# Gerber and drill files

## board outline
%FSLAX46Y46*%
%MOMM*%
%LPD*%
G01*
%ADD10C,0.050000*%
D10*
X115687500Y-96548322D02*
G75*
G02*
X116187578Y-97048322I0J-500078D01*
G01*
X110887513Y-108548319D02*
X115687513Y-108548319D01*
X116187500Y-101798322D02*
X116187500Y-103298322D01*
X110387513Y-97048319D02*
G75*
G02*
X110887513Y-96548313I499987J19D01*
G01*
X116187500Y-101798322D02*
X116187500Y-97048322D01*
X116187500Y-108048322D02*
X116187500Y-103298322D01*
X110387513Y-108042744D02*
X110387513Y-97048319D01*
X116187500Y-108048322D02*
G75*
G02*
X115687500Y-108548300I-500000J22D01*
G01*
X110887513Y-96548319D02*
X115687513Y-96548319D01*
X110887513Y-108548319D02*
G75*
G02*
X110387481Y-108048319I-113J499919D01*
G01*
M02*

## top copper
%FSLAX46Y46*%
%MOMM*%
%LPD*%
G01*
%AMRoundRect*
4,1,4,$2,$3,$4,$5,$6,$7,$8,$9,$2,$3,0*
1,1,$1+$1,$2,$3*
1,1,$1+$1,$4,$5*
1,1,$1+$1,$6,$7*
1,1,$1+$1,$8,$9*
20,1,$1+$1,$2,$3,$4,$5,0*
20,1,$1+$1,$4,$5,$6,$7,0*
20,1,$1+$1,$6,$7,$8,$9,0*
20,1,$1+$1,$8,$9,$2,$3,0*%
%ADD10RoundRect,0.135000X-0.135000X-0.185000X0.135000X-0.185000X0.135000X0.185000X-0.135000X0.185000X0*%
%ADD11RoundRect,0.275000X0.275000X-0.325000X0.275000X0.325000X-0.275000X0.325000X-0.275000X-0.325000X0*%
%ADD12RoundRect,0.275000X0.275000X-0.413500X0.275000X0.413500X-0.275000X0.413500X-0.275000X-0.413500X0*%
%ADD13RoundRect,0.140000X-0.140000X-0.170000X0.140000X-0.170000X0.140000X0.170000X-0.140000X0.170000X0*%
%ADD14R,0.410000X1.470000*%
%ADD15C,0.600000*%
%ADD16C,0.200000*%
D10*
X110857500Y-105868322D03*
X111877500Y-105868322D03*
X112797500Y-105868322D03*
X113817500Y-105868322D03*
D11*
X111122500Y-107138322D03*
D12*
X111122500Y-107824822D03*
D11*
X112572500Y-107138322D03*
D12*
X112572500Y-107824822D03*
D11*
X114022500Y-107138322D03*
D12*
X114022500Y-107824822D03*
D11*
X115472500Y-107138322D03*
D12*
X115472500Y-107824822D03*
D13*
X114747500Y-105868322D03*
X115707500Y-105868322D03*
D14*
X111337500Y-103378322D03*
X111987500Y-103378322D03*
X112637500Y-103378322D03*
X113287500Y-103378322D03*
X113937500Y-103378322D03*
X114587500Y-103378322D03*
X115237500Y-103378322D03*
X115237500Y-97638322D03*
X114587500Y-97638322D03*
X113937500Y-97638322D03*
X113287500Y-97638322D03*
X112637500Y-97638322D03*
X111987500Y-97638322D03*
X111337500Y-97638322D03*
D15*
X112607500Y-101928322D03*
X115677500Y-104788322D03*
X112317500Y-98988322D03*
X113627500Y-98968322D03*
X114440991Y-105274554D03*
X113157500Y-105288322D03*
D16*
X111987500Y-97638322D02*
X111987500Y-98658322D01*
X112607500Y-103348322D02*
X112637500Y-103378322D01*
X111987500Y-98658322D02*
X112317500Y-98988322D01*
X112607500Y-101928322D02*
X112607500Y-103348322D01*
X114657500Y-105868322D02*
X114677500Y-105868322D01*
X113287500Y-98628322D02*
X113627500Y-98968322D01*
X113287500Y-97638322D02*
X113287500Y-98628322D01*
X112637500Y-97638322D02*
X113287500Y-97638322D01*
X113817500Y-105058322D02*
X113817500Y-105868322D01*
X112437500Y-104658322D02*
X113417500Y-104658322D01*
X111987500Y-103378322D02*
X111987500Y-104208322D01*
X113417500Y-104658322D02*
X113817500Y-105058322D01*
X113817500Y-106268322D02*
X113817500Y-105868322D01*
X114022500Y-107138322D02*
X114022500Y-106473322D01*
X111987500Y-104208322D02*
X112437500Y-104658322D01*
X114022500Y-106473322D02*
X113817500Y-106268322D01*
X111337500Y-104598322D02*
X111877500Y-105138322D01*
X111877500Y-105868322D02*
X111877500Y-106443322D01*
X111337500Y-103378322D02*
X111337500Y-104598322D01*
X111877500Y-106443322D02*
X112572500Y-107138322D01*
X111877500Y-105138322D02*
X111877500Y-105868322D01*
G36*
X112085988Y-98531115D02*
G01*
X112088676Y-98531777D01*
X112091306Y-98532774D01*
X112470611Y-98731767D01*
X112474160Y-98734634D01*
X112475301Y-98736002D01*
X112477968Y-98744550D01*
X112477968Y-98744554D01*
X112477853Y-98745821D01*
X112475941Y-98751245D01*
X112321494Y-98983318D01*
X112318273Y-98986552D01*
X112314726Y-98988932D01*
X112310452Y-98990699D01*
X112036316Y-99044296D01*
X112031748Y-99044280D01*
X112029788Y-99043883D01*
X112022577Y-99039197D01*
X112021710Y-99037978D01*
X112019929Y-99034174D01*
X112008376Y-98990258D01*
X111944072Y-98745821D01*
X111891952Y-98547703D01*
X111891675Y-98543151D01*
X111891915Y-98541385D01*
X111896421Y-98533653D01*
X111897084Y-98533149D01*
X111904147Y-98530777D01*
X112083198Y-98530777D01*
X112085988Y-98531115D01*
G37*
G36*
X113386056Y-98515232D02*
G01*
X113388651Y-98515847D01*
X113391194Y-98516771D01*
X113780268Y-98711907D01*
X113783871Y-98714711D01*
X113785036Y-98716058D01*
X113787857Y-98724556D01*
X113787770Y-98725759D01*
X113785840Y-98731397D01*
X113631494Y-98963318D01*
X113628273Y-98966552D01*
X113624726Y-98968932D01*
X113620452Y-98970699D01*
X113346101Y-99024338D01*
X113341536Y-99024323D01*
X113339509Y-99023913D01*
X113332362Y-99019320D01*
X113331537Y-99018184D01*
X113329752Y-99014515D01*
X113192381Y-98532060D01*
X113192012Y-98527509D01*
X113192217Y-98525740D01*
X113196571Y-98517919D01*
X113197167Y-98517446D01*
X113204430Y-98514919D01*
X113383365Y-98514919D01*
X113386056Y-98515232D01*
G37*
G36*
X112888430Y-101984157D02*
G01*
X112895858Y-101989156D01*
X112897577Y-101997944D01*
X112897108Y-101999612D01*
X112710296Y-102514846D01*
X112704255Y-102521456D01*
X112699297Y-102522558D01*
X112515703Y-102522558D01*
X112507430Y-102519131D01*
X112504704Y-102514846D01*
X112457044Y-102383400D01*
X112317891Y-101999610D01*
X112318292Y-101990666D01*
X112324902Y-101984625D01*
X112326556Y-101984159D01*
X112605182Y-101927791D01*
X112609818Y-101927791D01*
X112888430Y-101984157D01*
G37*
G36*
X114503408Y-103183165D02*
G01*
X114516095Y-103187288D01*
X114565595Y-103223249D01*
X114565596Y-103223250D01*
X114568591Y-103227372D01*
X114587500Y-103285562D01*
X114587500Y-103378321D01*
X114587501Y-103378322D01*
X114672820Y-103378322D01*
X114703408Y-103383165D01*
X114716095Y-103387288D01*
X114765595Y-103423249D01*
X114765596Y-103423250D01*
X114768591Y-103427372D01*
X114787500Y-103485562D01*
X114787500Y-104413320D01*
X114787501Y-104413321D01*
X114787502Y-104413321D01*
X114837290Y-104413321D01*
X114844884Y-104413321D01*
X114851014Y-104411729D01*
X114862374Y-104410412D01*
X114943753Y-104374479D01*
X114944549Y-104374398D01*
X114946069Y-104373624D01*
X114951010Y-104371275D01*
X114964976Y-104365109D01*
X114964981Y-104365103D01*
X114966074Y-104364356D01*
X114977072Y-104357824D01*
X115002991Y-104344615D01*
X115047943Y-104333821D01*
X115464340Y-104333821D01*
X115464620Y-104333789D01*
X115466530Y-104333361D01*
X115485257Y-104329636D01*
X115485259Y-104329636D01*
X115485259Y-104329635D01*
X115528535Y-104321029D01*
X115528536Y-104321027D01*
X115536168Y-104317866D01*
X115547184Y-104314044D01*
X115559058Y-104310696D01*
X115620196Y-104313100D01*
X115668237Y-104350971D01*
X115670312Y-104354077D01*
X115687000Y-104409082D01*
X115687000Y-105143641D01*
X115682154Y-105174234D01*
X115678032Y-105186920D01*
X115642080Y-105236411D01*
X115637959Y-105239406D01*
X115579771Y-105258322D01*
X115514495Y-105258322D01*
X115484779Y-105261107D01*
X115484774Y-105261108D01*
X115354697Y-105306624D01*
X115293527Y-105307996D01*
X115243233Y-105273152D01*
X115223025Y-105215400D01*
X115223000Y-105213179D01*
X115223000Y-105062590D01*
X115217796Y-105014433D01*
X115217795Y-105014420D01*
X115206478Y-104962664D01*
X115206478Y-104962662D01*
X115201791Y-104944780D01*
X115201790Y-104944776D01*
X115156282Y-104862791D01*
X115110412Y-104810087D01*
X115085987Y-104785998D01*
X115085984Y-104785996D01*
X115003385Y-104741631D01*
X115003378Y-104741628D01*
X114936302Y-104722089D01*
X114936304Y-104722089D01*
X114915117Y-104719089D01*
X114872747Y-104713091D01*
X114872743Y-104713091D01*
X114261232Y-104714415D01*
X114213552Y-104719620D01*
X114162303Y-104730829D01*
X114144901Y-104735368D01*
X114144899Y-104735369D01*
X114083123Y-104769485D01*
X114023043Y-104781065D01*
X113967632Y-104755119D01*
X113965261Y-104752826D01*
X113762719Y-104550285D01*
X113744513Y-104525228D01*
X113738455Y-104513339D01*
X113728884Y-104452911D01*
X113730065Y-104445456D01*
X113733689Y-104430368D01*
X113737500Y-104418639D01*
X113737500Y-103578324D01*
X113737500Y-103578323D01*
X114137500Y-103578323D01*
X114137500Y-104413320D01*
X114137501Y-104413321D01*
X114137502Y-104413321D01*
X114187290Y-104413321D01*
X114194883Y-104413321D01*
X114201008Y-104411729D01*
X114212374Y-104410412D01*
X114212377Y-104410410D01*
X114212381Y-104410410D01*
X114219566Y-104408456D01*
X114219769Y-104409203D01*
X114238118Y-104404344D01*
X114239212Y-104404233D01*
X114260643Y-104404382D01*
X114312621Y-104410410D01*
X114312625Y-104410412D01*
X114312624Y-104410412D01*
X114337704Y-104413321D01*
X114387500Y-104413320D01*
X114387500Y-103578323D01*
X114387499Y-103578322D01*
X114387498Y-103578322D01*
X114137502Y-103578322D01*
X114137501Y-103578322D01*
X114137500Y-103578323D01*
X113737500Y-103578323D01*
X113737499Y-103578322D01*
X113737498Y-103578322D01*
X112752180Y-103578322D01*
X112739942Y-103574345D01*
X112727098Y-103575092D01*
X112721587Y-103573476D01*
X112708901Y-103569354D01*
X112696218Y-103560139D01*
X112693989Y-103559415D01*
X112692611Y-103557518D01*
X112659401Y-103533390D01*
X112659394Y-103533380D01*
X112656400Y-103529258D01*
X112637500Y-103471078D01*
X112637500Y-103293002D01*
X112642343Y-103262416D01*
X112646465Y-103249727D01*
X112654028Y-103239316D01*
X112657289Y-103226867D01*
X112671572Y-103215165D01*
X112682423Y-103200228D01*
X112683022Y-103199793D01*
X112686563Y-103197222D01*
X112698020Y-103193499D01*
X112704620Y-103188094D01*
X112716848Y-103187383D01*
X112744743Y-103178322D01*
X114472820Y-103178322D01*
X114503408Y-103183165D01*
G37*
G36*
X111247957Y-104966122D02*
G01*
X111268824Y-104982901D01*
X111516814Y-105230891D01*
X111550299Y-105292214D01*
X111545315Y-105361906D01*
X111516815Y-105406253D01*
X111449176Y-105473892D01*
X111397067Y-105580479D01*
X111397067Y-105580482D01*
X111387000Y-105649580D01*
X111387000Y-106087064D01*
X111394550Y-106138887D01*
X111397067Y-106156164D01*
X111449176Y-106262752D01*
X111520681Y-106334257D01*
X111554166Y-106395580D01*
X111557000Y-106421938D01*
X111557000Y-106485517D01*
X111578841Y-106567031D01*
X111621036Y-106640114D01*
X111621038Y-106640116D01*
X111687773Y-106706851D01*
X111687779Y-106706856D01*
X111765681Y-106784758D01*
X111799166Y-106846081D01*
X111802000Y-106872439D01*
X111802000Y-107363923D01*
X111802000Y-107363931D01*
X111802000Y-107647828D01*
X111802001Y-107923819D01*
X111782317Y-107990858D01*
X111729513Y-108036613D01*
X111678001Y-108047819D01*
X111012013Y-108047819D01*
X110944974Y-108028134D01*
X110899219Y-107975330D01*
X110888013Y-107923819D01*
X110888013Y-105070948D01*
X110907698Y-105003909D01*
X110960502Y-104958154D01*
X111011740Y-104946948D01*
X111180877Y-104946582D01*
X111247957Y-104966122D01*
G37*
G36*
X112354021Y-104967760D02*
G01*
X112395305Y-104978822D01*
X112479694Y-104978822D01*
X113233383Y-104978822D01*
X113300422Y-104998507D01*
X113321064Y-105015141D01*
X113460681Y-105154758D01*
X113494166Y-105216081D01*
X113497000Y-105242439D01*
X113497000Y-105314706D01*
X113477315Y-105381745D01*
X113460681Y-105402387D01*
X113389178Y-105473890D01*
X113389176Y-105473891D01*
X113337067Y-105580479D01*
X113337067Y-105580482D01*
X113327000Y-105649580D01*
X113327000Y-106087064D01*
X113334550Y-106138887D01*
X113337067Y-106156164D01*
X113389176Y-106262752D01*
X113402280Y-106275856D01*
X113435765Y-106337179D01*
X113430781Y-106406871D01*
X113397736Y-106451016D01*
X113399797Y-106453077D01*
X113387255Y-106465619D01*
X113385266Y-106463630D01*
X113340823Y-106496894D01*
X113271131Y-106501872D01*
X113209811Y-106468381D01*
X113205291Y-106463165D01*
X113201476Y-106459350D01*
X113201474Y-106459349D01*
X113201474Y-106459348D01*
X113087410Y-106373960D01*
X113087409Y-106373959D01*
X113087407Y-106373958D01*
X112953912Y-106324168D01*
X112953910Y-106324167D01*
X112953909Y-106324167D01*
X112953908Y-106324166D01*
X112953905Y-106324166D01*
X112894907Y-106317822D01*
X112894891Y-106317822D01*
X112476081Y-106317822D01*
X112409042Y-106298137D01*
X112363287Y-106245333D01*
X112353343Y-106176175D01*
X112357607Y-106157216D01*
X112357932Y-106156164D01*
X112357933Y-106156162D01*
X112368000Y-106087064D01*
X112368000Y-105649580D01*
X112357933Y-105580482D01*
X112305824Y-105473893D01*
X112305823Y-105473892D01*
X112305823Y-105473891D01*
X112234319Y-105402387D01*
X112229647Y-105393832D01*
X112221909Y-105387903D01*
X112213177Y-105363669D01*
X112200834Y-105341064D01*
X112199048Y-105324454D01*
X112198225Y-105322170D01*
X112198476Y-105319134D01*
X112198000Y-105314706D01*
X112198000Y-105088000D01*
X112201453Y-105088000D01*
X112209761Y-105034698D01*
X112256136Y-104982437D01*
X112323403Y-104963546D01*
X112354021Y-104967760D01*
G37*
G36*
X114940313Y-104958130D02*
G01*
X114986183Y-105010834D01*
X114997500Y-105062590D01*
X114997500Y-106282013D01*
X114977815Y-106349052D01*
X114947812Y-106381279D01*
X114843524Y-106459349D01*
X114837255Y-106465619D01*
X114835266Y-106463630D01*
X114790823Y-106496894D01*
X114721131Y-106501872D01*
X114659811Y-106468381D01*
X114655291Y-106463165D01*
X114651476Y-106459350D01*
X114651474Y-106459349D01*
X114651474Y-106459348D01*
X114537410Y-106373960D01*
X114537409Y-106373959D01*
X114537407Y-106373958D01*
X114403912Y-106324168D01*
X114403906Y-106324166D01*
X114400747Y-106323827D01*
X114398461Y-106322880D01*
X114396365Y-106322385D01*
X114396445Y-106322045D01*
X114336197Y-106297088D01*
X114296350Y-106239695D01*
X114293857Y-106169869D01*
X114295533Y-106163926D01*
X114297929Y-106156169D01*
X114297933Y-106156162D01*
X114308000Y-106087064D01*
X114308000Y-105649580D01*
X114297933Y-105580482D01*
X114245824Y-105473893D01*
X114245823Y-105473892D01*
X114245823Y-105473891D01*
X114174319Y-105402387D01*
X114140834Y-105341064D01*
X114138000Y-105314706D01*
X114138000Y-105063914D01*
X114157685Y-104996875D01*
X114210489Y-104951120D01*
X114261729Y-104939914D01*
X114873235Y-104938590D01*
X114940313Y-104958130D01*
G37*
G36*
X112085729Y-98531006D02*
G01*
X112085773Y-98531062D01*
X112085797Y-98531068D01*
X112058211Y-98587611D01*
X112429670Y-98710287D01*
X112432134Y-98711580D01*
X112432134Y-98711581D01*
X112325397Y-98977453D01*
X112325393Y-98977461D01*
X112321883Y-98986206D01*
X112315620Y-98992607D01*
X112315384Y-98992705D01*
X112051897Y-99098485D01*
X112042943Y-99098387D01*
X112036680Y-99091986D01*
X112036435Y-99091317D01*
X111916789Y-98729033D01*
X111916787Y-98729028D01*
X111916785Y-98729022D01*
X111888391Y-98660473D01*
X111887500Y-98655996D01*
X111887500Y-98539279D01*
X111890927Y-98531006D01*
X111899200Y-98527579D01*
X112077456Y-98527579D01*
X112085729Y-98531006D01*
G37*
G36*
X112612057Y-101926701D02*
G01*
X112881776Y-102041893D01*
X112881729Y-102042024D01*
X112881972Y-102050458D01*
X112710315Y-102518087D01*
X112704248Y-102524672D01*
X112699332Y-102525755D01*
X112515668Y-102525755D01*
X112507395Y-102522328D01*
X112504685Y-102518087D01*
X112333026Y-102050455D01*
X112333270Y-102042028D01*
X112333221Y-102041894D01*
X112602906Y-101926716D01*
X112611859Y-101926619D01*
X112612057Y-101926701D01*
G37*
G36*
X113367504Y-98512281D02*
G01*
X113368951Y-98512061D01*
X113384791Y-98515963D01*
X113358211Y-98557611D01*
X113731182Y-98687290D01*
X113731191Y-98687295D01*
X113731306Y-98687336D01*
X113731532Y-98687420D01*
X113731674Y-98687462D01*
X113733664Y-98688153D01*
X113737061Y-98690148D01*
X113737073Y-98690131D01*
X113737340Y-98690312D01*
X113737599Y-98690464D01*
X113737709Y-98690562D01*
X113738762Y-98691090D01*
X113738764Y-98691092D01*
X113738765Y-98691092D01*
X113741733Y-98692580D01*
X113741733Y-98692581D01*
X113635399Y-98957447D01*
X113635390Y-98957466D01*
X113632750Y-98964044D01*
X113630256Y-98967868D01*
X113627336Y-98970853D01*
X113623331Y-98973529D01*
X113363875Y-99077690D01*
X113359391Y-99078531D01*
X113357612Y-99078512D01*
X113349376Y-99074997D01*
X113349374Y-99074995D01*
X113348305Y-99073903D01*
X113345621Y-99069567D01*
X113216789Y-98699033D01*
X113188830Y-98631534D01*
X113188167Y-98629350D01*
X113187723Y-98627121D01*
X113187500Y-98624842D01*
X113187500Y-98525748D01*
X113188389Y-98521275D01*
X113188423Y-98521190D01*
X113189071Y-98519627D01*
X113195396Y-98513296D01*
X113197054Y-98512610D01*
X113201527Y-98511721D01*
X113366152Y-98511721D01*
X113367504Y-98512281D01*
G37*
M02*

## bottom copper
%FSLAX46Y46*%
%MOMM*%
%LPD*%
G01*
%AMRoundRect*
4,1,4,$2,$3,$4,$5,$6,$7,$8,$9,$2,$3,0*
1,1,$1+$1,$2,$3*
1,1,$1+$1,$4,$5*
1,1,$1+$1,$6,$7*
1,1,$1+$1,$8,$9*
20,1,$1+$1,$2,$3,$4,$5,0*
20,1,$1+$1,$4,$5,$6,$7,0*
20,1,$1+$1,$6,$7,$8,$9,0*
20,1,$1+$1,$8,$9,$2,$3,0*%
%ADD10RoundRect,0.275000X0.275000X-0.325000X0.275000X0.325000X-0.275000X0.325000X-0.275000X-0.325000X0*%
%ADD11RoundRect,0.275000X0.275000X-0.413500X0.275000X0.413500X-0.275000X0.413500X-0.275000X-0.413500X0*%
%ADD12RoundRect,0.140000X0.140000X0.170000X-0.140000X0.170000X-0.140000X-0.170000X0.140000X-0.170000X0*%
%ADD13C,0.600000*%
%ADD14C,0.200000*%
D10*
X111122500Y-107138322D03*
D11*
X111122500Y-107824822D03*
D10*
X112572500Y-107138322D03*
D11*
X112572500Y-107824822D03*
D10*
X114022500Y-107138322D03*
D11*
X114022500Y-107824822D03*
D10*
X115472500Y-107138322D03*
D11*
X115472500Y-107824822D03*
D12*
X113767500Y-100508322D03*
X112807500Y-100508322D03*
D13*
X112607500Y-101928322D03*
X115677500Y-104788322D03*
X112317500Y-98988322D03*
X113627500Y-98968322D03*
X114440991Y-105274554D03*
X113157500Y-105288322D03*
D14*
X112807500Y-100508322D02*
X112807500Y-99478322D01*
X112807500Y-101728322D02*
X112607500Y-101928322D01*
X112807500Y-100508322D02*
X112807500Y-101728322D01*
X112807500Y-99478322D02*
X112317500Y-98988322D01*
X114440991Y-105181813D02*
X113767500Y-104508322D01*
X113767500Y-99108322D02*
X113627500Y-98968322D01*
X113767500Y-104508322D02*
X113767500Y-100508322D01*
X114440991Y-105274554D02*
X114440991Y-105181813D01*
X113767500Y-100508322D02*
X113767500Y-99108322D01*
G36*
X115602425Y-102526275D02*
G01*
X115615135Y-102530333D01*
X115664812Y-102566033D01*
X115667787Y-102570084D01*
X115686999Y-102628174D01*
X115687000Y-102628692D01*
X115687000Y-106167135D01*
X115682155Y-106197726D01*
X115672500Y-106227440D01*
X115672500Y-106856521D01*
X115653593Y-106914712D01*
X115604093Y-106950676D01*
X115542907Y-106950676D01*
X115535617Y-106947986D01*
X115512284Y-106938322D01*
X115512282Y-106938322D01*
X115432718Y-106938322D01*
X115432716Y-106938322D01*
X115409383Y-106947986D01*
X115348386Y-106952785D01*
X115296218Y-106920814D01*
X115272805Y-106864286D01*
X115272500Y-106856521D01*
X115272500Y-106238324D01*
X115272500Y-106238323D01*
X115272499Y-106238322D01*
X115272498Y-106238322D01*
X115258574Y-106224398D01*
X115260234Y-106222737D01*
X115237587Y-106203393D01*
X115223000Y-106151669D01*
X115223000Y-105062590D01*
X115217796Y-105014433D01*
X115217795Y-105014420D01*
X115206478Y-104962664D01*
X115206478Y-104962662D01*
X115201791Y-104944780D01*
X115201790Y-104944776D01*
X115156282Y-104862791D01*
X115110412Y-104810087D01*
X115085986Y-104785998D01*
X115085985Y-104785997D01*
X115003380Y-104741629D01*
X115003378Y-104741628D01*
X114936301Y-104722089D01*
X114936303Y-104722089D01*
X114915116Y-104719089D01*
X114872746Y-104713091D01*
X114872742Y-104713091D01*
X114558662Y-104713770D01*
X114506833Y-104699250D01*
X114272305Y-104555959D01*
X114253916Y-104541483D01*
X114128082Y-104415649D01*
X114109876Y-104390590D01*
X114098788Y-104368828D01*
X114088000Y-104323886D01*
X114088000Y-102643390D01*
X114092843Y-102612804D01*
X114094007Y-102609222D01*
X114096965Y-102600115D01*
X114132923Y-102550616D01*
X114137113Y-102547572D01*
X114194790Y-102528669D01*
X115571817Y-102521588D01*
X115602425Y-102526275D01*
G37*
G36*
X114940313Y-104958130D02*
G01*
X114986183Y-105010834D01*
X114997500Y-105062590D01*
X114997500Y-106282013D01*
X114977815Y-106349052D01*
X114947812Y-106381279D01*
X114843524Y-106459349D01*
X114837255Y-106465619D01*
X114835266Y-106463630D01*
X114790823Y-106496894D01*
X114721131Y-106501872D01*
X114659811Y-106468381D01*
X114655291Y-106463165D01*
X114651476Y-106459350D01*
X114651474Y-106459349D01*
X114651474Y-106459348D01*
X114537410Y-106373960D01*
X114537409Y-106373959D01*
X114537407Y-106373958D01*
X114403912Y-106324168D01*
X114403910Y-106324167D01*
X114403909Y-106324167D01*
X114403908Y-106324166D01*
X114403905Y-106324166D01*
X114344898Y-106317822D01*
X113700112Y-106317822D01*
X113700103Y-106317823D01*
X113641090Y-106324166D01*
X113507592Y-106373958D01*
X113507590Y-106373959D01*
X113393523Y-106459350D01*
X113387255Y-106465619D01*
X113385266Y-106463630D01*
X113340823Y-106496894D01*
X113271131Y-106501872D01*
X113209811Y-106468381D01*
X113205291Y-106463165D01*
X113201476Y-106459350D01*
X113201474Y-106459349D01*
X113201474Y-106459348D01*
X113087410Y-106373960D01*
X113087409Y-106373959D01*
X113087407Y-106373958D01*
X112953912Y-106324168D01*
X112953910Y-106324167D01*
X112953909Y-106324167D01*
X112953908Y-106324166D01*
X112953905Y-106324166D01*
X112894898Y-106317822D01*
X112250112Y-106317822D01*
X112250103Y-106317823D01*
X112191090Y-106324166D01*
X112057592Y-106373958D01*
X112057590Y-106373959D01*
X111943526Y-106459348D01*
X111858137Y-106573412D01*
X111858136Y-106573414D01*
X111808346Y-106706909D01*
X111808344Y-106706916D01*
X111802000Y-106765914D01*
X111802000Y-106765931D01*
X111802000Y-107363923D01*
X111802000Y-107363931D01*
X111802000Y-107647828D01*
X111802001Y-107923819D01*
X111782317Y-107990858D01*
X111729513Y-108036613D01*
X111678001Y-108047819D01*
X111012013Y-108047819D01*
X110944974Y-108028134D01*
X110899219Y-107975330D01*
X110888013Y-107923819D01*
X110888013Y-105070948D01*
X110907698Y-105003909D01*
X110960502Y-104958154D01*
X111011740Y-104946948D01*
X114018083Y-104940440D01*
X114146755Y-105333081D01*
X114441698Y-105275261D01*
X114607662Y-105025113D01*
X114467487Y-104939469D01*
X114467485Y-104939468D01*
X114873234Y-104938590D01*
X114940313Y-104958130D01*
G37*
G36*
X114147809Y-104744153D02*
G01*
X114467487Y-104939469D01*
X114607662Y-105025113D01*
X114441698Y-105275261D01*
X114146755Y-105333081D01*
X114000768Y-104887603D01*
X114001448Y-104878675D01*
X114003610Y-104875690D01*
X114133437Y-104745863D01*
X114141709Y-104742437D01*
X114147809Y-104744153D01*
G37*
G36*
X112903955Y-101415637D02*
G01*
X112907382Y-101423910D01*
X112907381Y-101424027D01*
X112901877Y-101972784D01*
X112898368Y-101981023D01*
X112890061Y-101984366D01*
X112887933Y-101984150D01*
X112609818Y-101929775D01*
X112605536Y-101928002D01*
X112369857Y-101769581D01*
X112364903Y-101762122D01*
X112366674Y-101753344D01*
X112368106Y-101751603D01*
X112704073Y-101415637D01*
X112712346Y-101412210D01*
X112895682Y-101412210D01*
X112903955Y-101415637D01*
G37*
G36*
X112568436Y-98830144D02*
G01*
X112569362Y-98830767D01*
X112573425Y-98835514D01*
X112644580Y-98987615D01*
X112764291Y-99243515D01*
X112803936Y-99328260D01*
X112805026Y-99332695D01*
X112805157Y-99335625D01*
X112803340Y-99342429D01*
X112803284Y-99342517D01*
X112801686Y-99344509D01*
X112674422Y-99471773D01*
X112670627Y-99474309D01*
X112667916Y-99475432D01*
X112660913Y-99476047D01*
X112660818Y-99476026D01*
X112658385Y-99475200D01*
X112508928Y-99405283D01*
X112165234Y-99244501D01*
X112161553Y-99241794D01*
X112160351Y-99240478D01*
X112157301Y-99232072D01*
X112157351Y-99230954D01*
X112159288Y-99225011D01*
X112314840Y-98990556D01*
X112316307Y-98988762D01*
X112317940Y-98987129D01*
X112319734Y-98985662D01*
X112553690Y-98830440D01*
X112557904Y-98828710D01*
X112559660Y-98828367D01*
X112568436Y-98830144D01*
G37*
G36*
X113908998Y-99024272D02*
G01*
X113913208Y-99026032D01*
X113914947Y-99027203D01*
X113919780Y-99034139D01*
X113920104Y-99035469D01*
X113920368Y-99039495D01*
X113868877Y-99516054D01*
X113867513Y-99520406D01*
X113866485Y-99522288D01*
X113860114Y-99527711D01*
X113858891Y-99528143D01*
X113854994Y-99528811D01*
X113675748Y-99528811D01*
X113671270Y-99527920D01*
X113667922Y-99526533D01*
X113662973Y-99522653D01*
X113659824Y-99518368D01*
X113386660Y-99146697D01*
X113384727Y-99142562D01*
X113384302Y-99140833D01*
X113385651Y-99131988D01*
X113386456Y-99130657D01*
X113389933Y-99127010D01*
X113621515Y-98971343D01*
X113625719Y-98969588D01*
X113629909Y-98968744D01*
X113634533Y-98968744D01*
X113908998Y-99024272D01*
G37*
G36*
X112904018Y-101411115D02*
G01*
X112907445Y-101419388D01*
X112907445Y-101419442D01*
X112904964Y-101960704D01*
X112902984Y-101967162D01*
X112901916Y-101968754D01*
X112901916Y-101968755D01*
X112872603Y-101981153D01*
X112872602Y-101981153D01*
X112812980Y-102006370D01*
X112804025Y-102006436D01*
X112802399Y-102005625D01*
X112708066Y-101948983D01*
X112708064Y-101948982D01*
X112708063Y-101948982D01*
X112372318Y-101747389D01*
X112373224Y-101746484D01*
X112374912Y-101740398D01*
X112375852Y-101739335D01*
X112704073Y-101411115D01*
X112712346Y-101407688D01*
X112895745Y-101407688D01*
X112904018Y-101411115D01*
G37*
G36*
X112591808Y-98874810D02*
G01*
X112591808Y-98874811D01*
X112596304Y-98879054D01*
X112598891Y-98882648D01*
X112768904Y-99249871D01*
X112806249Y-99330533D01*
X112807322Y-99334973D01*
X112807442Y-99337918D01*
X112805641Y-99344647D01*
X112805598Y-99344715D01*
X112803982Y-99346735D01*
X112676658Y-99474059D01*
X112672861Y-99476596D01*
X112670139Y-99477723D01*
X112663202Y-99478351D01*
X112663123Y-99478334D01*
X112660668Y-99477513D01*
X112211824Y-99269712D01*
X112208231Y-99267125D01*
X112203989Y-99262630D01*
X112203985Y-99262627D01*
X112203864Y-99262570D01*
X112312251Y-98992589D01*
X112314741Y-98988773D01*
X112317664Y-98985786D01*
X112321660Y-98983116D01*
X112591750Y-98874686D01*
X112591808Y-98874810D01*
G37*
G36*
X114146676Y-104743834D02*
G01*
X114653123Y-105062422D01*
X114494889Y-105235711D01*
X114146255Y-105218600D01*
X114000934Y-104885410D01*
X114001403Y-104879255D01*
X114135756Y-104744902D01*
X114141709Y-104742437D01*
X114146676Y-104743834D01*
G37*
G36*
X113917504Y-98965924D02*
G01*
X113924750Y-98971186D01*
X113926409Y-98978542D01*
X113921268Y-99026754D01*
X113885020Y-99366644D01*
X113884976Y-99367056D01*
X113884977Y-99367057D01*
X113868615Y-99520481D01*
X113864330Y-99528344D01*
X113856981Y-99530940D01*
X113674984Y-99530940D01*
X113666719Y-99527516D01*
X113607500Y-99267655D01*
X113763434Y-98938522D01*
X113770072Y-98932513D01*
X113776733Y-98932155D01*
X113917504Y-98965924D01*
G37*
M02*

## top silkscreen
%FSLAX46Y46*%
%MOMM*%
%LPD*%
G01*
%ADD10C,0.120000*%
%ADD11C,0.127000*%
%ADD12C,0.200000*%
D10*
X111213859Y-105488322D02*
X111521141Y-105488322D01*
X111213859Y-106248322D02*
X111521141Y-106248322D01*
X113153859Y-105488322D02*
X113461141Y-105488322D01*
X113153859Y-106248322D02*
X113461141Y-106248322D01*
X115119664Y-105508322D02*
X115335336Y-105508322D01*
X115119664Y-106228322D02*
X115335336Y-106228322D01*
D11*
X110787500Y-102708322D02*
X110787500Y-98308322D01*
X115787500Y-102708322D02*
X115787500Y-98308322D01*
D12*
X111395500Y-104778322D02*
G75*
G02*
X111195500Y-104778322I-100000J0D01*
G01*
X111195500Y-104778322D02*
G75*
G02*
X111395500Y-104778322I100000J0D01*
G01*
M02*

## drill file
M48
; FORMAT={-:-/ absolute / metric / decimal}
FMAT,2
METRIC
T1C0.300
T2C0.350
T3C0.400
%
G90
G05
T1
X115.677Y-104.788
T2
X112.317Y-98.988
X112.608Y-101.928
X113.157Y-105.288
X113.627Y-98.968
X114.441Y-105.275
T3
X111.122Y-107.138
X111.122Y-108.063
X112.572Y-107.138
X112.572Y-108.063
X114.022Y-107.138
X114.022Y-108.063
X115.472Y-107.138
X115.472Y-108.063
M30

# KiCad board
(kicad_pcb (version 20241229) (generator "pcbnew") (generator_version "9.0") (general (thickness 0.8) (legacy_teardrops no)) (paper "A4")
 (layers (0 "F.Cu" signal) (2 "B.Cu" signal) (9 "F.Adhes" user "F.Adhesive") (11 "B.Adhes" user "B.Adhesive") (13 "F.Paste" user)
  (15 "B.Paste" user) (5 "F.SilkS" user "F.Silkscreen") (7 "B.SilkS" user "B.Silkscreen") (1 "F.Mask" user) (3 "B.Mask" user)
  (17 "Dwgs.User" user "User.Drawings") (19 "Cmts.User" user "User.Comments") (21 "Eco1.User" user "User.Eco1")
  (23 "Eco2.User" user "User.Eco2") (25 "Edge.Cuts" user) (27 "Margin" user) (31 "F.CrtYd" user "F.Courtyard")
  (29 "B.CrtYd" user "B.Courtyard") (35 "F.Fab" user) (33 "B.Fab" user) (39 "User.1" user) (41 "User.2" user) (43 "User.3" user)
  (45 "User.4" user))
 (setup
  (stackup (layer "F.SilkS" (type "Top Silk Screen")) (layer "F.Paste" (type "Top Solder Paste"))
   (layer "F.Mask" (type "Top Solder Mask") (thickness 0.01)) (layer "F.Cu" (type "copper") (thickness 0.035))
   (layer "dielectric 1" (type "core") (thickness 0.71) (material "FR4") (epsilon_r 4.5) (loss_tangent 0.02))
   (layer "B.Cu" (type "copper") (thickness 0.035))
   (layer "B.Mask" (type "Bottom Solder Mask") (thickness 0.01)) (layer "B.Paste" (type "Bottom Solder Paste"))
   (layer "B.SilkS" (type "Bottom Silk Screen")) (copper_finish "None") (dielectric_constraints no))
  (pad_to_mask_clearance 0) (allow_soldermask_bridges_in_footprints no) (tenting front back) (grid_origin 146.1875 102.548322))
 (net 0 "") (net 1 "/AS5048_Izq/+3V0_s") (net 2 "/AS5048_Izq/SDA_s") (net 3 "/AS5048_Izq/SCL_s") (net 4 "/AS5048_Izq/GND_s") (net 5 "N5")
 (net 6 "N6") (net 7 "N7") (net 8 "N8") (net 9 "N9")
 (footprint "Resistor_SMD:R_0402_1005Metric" (layer "F.Cu") (at 111.3675 105.868322)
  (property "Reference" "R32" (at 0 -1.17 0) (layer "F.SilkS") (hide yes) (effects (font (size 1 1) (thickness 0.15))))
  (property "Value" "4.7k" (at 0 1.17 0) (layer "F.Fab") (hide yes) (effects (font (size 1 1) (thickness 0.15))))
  (fp_line (start -0.153641 -0.38) (end 0.153641 -0.38) (stroke (width 0.12) (type solid)) (layer "F.SilkS"))
  (fp_line (start -0.153641 0.38) (end 0.153641 0.38) (stroke (width 0.12) (type solid)) (layer "F.SilkS"))
  (pad "1" smd roundrect (at -0.51 0) (size 0.54 0.64) (layers "F.Cu" "F.Mask" "F.Paste") (roundrect_rratio 0.25)
   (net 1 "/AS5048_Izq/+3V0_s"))
  (pad "2" smd roundrect (at 0.51 0) (size 0.54 0.64) (layers "F.Cu" "F.Mask" "F.Paste") (roundrect_rratio 0.25) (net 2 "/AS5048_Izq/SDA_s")))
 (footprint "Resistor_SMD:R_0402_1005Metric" (layer "F.Cu") (at 113.3075 105.868322)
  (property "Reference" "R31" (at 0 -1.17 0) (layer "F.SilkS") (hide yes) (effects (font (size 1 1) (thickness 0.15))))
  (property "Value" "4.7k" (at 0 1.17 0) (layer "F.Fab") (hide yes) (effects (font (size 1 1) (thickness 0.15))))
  (fp_line (start -0.153641 -0.38) (end 0.153641 -0.38) (stroke (width 0.12) (type solid)) (layer "F.SilkS"))
  (fp_line (start -0.153641 0.38) (end 0.153641 0.38) (stroke (width 0.12) (type solid)) (layer "F.SilkS"))
  (pad "1" smd roundrect (at -0.51 0) (size 0.54 0.64) (layers "F.Cu" "F.Mask" "F.Paste") (roundrect_rratio 0.25)
   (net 1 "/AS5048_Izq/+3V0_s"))
  (pad "2" smd roundrect (at 0.51 0) (size 0.54 0.64) (layers "F.Cu" "F.Mask" "F.Paste") (roundrect_rratio 0.25) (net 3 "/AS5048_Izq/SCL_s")))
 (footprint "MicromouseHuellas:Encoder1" (layer "F.Cu") (at 113.2975 107.138322)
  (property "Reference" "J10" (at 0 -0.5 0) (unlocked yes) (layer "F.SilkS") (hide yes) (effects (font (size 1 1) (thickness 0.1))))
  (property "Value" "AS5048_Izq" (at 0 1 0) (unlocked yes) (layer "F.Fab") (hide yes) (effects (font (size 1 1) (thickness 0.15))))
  (pad "1" thru_hole roundrect (at -2.175 0 90) (size 1.2 1.1) (drill 0.4) (layers "*.Cu" "*.Mask") (remove_unused_layers no)
   (roundrect_rratio 0.25) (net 1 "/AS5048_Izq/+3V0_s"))
  (pad "1" thru_hole roundrect (at -2.175 0.925 90) (size 1.377 1.1) (drill 0.4 (offset 0.2385 0)) (layers "*.Cu" "*.Mask")
   (remove_unused_layers no) (roundrect_rratio 0.25) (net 1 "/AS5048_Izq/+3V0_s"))
  (pad "2" thru_hole roundrect (at -0.725 0 90) (size 1.2 1.1) (drill 0.4) (layers "*.Cu" "*.Mask") (remove_unused_layers no)
   (roundrect_rratio 0.25) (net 2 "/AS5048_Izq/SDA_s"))
  (pad "2" thru_hole roundrect (at -0.725 0.925 90) (size 1.377 1.1) (drill 0.4 (offset 0.2385 0)) (layers "*.Cu" "*.Mask")
   (remove_unused_layers no) (roundrect_rratio 0.25) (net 2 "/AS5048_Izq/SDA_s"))
  (pad "3" thru_hole roundrect (at 0.725 0 90) (size 1.2 1.1) (drill 0.4) (layers "*.Cu" "*.Mask") (remove_unused_layers no)
   (roundrect_rratio 0.25) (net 3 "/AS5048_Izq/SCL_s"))
  (pad "3" thru_hole roundrect (at 0.725 0.925 90) (size 1.377 1.1) (drill 0.4 (offset 0.2385 0)) (layers "*.Cu" "*.Mask")
   (remove_unused_layers no) (roundrect_rratio 0.25) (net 3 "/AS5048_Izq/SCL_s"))
  (pad "4" thru_hole roundrect (at 2.175 0 90) (size 1.2 1.1) (drill 0.4) (layers "*.Cu" "*.Mask") (remove_unused_layers no)
   (roundrect_rratio 0.25) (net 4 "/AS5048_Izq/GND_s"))
  (pad "4" thru_hole roundrect (at 2.175 0.925 90) (size 1.377 1.1) (drill 0.4 (offset 0.2385 0)) (layers "*.Cu" "*.Mask")
   (remove_unused_layers no) (roundrect_rratio 0.25) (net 4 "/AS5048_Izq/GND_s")))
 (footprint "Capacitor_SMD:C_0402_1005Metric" (layer "F.Cu") (at 115.2275 105.868322)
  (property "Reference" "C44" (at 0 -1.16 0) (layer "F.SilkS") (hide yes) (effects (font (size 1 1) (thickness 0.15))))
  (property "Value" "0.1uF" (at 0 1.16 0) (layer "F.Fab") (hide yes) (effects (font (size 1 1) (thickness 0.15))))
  (fp_line (start -0.107836 -0.36) (end 0.107836 -0.36) (stroke (width 0.12) (type solid)) (layer "F.SilkS"))
  (fp_line (start -0.107836 0.36) (end 0.107836 0.36) (stroke (width 0.12) (type solid)) (layer "F.SilkS"))
  (pad "1" smd roundrect (at -0.48 0) (size 0.56 0.62) (layers "F.Cu" "F.Mask" "F.Paste") (roundrect_rratio 0.25)
   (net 1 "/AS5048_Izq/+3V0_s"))
  (pad "2" smd roundrect (at 0.48 0) (size 0.56 0.62) (layers "F.Cu" "F.Mask" "F.Paste") (roundrect_rratio 0.25) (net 4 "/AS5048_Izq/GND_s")))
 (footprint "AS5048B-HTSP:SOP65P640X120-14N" (layer "F.Cu") (at 113.2875 100.508322 90)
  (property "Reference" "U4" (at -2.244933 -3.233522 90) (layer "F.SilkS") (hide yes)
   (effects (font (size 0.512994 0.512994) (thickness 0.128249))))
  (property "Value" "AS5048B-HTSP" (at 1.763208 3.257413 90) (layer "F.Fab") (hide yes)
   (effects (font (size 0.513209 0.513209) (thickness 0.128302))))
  (fp_line (start -2.2 -2.5) (end 2.2 -2.5) (stroke (width 0.127) (type solid)) (layer "F.SilkS"))
  (fp_line (start -2.2 2.5) (end 2.2 2.5) (stroke (width 0.127) (type solid)) (layer "F.SilkS"))
  (fp_circle (center -4.27 -1.992) (end -4.17 -1.992) (stroke (width 0.2) (type solid)) (fill no) (layer "F.SilkS"))
  (pad "1" smd rect (at -2.87 -1.95 90) (size 1.47 0.41) (layers "F.Cu" "F.Mask" "F.Paste") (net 2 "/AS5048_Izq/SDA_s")
   (solder_mask_margin 0.102))
  (pad "2" smd rect (at -2.87 -1.3 90) (size 1.47 0.41) (layers "F.Cu" "F.Mask" "F.Paste") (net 3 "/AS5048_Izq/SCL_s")
   (solder_mask_margin 0.102))
  (pad "3" smd rect (at -2.87 -0.65 90) (size 1.47 0.41) (layers "F.Cu" "F.Mask" "F.Paste") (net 4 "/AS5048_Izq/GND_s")
   (solder_mask_margin 0.102))
  (pad "4" smd rect (at -2.87 0 90) (size 1.47 0.41) (layers "F.Cu" "F.Mask" "F.Paste") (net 4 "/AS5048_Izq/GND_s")
   (solder_mask_margin 0.102))
  (pad "5" smd rect (at -2.87 0.65 90) (size 1.47 0.41) (layers "F.Cu" "F.Mask" "F.Paste") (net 4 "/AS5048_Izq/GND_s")
   (solder_mask_margin 0.102))
  (pad "6" smd rect (at -2.87 1.3 90) (size 1.47 0.41) (layers "F.Cu" "F.Mask" "F.Paste") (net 4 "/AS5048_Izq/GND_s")
   (solder_mask_margin 0.102))
  (pad "7" smd rect (at -2.87 1.95 90) (size 1.47 0.41) (layers "F.Cu" "F.Mask" "F.Paste") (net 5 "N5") (solder_mask_margin 0.102))
  (pad "8" smd rect (at 2.87 1.95 90) (size 1.47 0.41) (layers "F.Cu" "F.Mask" "F.Paste") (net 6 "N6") (solder_mask_margin 0.102))
  (pad "9" smd rect (at 2.87 1.3 90) (size 1.47 0.41) (layers "F.Cu" "F.Mask" "F.Paste") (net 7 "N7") (solder_mask_margin 0.102))
  (pad "10" smd rect (at 2.87 0.65 90) (size 1.47 0.41) (layers "F.Cu" "F.Mask" "F.Paste") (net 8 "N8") (solder_mask_margin 0.102))
  (pad "11" smd rect (at 2.87 0 90) (size 1.47 0.41) (layers "F.Cu" "F.Mask" "F.Paste") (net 1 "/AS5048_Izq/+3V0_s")
   (solder_mask_margin 0.102))
  (pad "12" smd rect (at 2.87 -0.65 90) (size 1.47 0.41) (layers "F.Cu" "F.Mask" "F.Paste") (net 1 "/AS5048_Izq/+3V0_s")
   (solder_mask_margin 0.102))
  (pad "13" smd rect (at 2.87 -1.3 90) (size 1.47 0.41) (layers "F.Cu" "F.Mask" "F.Paste") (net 4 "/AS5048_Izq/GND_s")
   (solder_mask_margin 0.102))
  (pad "14" smd rect (at 2.87 -1.95 90) (size 1.47 0.41) (layers "F.Cu" "F.Mask" "F.Paste") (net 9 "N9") (solder_mask_margin 0.102)))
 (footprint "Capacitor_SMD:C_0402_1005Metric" (layer "B.Cu") (at 113.2875 100.508322 180)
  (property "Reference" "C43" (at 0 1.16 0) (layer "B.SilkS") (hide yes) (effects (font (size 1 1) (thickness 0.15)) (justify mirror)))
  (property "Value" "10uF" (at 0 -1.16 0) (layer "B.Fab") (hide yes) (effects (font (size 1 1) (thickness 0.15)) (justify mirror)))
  (pad "1" smd roundrect (at -0.48 0 180) (size 0.56 0.62) (layers "B.Cu" "B.Mask" "B.Paste") (roundrect_rratio 0.25)
   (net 1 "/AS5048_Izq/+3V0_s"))
  (pad "2" smd roundrect (at 0.48 0 180) (size 0.56 0.62) (layers "B.Cu" "B.Mask" "B.Paste") (roundrect_rratio 0.25)
   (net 4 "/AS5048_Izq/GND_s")))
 (gr_arc (start 115.6875 96.548322) (mid 116.041031 96.694772) (end 116.1875 97.048322) (stroke (width 0.05) (type default))
  (layer "Edge.Cuts"))
 (gr_line (start 110.887513 108.548319) (end 115.687513 108.548319) (stroke (width 0.05) (type solid)) (layer "Edge.Cuts"))
 (gr_line (start 116.1875 101.798322) (end 116.1875 103.298322) (stroke (width 0.05) (type default)) (layer "Edge.Cuts"))
 (gr_arc (start 110.387513 97.048319) (mid 110.533968 96.69476) (end 110.887513 96.548319) (stroke (width 0.05) (type default))
  (layer "Edge.Cuts"))
 (gr_line (start 116.1875 101.798322) (end 116.1875 97.048322) (stroke (width 0.05) (type solid)) (layer "Edge.Cuts"))
 (gr_line (start 116.1875 108.048322) (end 116.1875 103.298322) (stroke (width 0.05) (type solid)) (layer "Edge.Cuts"))
 (gr_line (start 110.387513 108.042744) (end 110.387513 97.048319) (stroke (width 0.05) (type default)) (layer "Edge.Cuts"))
 (gr_arc (start 116.1875 108.048322) (mid 116.04106 108.401863) (end 115.6875 108.548322) (stroke (width 0.05) (type default))
  (layer "Edge.Cuts"))
 (gr_line (start 110.887513 96.548319) (end 115.687513 96.548319) (stroke (width 0.05) (type solid)) (layer "Edge.Cuts"))
 (gr_arc (start 110.887513 108.548319) (mid 110.53393 108.401881) (end 110.387513 108.048319) (stroke (width 0.05) (type default))
  (layer "Edge.Cuts"))
 (segment (start 111.9875 97.638322) (end 111.9875 98.658322) (width 0.2) (layer "F.Cu") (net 4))
 (segment (start 112.6075 103.348322) (end 112.6375 103.378322) (width 0.2) (layer "F.Cu") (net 4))
 (segment (start 111.9875 98.658322) (end 112.3175 98.988322) (width 0.2) (layer "F.Cu") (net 4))
 (segment (start 112.6075 101.928322) (end 112.6075 103.348322) (width 0.2) (layer "F.Cu") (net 4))
 (via (at 112.6075 101.928322) (size 0.6) (drill 0.35) (layers "F.Cu" "B.Cu")
  (teardrops (best_length_ratio 0.5) (max_length 1) (best_width_ratio 1) (max_width 2) (curved_edges no) (filter_ratio 0.9) (enabled yes)
   (allow_two_segments yes) (prefer_zone_connections yes))
  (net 4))
 (via (at 115.6775 104.788322) (size 0.6) (drill 0.3) (layers "F.Cu" "B.Cu") (free yes) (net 4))
 (via (at 112.3175 98.988322) (size 0.6) (drill 0.35) (layers "F.Cu" "B.Cu")
  (teardrops (best_length_ratio 0.5) (max_length 1) (best_width_ratio 1) (max_width 2) (curved_edges no) (filter_ratio 0.9) (enabled yes)
   (allow_two_segments yes) (prefer_zone_connections yes))
  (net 4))
 (segment (start 112.8075 100.508322) (end 112.8075 99.478322) (width 0.2) (layer "B.Cu") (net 4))
 (segment (start 112.8075 101.728322) (end 112.6075 101.928322) (width 0.2) (layer "B.Cu") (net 4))
 (segment (start 112.8075 100.508322) (end 112.8075 101.728322) (width 0.2) (layer "B.Cu") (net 4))
 (segment (start 112.8075 99.478322) (end 112.3175 98.988322) (width 0.2) (layer "B.Cu") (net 4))
 (segment (start 114.6575 105.868322) (end 114.6775 105.868322) (width 0.2) (layer "F.Cu") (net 1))
 (segment (start 113.2875 98.628322) (end 113.6275 98.968322) (width 0.2) (layer "F.Cu") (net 1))
 (segment (start 113.2875 97.638322) (end 113.2875 98.628322) (width 0.2) (layer "F.Cu") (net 1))
 (segment (start 112.6375 97.638322) (end 113.2875 97.638322) (width 0.2) (layer "F.Cu") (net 1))
 (via (at 113.6275 98.968322) (size 0.6) (drill 0.35) (layers "F.Cu" "B.Cu")
  (teardrops (best_length_ratio 0.5) (max_length 1) (best_width_ratio 1) (max_width 2) (curved_edges no) (filter_ratio 0.9) (enabled yes)
   (allow_two_segments yes) (prefer_zone_connections yes))
  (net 1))
 (via (at 114.440991 105.274554) (size 0.6) (drill 0.35) (layers "F.Cu" "B.Cu")
  (teardrops (best_length_ratio 0.5) (max_length 1) (best_width_ratio 1) (max_width 2) (curved_edges no) (filter_ratio 0.9) (enabled yes)
   (allow_two_segments yes) (prefer_zone_connections yes))
  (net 1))
 (via (at 113.1575 105.288322) (size 0.6) (drill 0.35) (layers "F.Cu" "B.Cu") (free yes)
  (teardrops (best_length_ratio 0.5) (max_length 1) (best_width_ratio 1) (max_width 2) (curved_edges no) (filter_ratio 0.9) (enabled yes)
   (allow_two_segments yes) (prefer_zone_connections yes))
  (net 1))
 (segment (start 114.440991 105.181813) (end 113.7675 104.508322) (width 0.2) (layer "B.Cu") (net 1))
 (segment (start 113.7675 99.108322) (end 113.6275 98.968322) (width 0.2) (layer "B.Cu") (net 1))
 (segment (start 113.7675 104.508322) (end 113.7675 100.508322) (width 0.2) (layer "B.Cu") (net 1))
 (segment (start 114.440991 105.274554) (end 114.440991 105.181813) (width 0.2) (layer "B.Cu") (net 1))
 (segment (start 113.7675 100.508322) (end 113.7675 99.108322) (width 0.2) (layer "B.Cu") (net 1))
 (segment (start 113.8175 105.058322) (end 113.8175 105.868322) (width 0.2) (layer "F.Cu") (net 3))
 (segment (start 112.4375 104.658322) (end 113.4175 104.658322) (width 0.2) (layer "F.Cu") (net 3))
 (segment (start 111.9875 103.378322) (end 111.9875 104.208322) (width 0.2) (layer "F.Cu") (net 3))
 (segment (start 113.4175 104.658322) (end 113.8175 105.058322) (width 0.2) (layer "F.Cu") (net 3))
 (segment (start 113.8175 106.268322) (end 113.8175 105.868322) (width 0.2) (layer "F.Cu") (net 3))
 (segment (start 114.0225 107.138322) (end 114.0225 106.473322) (width 0.2) (layer "F.Cu") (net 3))
 (segment (start 111.9875 104.208322) (end 112.4375 104.658322) (width 0.2) (layer "F.Cu") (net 3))
 (segment (start 114.0225 106.473322) (end 113.8175 106.268322) (width 0.2) (layer "F.Cu") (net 3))
 (segment (start 111.3375 104.598322) (end 111.8775 105.138322) (width 0.2) (layer "F.Cu") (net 2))
 (segment (start 111.8775 105.868322) (end 111.8775 106.443322) (width 0.2) (layer "F.Cu") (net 2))
 (segment (start 111.3375 103.378322) (end 111.3375 104.598322) (width 0.2) (layer "F.Cu") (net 2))
 (segment (start 111.8775 106.443322) (end 112.5725 107.138322) (width 0.2) (layer "F.Cu") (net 2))
 (segment (start 111.8775 105.138322) (end 111.8775 105.868322) (width 0.2) (layer "F.Cu") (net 2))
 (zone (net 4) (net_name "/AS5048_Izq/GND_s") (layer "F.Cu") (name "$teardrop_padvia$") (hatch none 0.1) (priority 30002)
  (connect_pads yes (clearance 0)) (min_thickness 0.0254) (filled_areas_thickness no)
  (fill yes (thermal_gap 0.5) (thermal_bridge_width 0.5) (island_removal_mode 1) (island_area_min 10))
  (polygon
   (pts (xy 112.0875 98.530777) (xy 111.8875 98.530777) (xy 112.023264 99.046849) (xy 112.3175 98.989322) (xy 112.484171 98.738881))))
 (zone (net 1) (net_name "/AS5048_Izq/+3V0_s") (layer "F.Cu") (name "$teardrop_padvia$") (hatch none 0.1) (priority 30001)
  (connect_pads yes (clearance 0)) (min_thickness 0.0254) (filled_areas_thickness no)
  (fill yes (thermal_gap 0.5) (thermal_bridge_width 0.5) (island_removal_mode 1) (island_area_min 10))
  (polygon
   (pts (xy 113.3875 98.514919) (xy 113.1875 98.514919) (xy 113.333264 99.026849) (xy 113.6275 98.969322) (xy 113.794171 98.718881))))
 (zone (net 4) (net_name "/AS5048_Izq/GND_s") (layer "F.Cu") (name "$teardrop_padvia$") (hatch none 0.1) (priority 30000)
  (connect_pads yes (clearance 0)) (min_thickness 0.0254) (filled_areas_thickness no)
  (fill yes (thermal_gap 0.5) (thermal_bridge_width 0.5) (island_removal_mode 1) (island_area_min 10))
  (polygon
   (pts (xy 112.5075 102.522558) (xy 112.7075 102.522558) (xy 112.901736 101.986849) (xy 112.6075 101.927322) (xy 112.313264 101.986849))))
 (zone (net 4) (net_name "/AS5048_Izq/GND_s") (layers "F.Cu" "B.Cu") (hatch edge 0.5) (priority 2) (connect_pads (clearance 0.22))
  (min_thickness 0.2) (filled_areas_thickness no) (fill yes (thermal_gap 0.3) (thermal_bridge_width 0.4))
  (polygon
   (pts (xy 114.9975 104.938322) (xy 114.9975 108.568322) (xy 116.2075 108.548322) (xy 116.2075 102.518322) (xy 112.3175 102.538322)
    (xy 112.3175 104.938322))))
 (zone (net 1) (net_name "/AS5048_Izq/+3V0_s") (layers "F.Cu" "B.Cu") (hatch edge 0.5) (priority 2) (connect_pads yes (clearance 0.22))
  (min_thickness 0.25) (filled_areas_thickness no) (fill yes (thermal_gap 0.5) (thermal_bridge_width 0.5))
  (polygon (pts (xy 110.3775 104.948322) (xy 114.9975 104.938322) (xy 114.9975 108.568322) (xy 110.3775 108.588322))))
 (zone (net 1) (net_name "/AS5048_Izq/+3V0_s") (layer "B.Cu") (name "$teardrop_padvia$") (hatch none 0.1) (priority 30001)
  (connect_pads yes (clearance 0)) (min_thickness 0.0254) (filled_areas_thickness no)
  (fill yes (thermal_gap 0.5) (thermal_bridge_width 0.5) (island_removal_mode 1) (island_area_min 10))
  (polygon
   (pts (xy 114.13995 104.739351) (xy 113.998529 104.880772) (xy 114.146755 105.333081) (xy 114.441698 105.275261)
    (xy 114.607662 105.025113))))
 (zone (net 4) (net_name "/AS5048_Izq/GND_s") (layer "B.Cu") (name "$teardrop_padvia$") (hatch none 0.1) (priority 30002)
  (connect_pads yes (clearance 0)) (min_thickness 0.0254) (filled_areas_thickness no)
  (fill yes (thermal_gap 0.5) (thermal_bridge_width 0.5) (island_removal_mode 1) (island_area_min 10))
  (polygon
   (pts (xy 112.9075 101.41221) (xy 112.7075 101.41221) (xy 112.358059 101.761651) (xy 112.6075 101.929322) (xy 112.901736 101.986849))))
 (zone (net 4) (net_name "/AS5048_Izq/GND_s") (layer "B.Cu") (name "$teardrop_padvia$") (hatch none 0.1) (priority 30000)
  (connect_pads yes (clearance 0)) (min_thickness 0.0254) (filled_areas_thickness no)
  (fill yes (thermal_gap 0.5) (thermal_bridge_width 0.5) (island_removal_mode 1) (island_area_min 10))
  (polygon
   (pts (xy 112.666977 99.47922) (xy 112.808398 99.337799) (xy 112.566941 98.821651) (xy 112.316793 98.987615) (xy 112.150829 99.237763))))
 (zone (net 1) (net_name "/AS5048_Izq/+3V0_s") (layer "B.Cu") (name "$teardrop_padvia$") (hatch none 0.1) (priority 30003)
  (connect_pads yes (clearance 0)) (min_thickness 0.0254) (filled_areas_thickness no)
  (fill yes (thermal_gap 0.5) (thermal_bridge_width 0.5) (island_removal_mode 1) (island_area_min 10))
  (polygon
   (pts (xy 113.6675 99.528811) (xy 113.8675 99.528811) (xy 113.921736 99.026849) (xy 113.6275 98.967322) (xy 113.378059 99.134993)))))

